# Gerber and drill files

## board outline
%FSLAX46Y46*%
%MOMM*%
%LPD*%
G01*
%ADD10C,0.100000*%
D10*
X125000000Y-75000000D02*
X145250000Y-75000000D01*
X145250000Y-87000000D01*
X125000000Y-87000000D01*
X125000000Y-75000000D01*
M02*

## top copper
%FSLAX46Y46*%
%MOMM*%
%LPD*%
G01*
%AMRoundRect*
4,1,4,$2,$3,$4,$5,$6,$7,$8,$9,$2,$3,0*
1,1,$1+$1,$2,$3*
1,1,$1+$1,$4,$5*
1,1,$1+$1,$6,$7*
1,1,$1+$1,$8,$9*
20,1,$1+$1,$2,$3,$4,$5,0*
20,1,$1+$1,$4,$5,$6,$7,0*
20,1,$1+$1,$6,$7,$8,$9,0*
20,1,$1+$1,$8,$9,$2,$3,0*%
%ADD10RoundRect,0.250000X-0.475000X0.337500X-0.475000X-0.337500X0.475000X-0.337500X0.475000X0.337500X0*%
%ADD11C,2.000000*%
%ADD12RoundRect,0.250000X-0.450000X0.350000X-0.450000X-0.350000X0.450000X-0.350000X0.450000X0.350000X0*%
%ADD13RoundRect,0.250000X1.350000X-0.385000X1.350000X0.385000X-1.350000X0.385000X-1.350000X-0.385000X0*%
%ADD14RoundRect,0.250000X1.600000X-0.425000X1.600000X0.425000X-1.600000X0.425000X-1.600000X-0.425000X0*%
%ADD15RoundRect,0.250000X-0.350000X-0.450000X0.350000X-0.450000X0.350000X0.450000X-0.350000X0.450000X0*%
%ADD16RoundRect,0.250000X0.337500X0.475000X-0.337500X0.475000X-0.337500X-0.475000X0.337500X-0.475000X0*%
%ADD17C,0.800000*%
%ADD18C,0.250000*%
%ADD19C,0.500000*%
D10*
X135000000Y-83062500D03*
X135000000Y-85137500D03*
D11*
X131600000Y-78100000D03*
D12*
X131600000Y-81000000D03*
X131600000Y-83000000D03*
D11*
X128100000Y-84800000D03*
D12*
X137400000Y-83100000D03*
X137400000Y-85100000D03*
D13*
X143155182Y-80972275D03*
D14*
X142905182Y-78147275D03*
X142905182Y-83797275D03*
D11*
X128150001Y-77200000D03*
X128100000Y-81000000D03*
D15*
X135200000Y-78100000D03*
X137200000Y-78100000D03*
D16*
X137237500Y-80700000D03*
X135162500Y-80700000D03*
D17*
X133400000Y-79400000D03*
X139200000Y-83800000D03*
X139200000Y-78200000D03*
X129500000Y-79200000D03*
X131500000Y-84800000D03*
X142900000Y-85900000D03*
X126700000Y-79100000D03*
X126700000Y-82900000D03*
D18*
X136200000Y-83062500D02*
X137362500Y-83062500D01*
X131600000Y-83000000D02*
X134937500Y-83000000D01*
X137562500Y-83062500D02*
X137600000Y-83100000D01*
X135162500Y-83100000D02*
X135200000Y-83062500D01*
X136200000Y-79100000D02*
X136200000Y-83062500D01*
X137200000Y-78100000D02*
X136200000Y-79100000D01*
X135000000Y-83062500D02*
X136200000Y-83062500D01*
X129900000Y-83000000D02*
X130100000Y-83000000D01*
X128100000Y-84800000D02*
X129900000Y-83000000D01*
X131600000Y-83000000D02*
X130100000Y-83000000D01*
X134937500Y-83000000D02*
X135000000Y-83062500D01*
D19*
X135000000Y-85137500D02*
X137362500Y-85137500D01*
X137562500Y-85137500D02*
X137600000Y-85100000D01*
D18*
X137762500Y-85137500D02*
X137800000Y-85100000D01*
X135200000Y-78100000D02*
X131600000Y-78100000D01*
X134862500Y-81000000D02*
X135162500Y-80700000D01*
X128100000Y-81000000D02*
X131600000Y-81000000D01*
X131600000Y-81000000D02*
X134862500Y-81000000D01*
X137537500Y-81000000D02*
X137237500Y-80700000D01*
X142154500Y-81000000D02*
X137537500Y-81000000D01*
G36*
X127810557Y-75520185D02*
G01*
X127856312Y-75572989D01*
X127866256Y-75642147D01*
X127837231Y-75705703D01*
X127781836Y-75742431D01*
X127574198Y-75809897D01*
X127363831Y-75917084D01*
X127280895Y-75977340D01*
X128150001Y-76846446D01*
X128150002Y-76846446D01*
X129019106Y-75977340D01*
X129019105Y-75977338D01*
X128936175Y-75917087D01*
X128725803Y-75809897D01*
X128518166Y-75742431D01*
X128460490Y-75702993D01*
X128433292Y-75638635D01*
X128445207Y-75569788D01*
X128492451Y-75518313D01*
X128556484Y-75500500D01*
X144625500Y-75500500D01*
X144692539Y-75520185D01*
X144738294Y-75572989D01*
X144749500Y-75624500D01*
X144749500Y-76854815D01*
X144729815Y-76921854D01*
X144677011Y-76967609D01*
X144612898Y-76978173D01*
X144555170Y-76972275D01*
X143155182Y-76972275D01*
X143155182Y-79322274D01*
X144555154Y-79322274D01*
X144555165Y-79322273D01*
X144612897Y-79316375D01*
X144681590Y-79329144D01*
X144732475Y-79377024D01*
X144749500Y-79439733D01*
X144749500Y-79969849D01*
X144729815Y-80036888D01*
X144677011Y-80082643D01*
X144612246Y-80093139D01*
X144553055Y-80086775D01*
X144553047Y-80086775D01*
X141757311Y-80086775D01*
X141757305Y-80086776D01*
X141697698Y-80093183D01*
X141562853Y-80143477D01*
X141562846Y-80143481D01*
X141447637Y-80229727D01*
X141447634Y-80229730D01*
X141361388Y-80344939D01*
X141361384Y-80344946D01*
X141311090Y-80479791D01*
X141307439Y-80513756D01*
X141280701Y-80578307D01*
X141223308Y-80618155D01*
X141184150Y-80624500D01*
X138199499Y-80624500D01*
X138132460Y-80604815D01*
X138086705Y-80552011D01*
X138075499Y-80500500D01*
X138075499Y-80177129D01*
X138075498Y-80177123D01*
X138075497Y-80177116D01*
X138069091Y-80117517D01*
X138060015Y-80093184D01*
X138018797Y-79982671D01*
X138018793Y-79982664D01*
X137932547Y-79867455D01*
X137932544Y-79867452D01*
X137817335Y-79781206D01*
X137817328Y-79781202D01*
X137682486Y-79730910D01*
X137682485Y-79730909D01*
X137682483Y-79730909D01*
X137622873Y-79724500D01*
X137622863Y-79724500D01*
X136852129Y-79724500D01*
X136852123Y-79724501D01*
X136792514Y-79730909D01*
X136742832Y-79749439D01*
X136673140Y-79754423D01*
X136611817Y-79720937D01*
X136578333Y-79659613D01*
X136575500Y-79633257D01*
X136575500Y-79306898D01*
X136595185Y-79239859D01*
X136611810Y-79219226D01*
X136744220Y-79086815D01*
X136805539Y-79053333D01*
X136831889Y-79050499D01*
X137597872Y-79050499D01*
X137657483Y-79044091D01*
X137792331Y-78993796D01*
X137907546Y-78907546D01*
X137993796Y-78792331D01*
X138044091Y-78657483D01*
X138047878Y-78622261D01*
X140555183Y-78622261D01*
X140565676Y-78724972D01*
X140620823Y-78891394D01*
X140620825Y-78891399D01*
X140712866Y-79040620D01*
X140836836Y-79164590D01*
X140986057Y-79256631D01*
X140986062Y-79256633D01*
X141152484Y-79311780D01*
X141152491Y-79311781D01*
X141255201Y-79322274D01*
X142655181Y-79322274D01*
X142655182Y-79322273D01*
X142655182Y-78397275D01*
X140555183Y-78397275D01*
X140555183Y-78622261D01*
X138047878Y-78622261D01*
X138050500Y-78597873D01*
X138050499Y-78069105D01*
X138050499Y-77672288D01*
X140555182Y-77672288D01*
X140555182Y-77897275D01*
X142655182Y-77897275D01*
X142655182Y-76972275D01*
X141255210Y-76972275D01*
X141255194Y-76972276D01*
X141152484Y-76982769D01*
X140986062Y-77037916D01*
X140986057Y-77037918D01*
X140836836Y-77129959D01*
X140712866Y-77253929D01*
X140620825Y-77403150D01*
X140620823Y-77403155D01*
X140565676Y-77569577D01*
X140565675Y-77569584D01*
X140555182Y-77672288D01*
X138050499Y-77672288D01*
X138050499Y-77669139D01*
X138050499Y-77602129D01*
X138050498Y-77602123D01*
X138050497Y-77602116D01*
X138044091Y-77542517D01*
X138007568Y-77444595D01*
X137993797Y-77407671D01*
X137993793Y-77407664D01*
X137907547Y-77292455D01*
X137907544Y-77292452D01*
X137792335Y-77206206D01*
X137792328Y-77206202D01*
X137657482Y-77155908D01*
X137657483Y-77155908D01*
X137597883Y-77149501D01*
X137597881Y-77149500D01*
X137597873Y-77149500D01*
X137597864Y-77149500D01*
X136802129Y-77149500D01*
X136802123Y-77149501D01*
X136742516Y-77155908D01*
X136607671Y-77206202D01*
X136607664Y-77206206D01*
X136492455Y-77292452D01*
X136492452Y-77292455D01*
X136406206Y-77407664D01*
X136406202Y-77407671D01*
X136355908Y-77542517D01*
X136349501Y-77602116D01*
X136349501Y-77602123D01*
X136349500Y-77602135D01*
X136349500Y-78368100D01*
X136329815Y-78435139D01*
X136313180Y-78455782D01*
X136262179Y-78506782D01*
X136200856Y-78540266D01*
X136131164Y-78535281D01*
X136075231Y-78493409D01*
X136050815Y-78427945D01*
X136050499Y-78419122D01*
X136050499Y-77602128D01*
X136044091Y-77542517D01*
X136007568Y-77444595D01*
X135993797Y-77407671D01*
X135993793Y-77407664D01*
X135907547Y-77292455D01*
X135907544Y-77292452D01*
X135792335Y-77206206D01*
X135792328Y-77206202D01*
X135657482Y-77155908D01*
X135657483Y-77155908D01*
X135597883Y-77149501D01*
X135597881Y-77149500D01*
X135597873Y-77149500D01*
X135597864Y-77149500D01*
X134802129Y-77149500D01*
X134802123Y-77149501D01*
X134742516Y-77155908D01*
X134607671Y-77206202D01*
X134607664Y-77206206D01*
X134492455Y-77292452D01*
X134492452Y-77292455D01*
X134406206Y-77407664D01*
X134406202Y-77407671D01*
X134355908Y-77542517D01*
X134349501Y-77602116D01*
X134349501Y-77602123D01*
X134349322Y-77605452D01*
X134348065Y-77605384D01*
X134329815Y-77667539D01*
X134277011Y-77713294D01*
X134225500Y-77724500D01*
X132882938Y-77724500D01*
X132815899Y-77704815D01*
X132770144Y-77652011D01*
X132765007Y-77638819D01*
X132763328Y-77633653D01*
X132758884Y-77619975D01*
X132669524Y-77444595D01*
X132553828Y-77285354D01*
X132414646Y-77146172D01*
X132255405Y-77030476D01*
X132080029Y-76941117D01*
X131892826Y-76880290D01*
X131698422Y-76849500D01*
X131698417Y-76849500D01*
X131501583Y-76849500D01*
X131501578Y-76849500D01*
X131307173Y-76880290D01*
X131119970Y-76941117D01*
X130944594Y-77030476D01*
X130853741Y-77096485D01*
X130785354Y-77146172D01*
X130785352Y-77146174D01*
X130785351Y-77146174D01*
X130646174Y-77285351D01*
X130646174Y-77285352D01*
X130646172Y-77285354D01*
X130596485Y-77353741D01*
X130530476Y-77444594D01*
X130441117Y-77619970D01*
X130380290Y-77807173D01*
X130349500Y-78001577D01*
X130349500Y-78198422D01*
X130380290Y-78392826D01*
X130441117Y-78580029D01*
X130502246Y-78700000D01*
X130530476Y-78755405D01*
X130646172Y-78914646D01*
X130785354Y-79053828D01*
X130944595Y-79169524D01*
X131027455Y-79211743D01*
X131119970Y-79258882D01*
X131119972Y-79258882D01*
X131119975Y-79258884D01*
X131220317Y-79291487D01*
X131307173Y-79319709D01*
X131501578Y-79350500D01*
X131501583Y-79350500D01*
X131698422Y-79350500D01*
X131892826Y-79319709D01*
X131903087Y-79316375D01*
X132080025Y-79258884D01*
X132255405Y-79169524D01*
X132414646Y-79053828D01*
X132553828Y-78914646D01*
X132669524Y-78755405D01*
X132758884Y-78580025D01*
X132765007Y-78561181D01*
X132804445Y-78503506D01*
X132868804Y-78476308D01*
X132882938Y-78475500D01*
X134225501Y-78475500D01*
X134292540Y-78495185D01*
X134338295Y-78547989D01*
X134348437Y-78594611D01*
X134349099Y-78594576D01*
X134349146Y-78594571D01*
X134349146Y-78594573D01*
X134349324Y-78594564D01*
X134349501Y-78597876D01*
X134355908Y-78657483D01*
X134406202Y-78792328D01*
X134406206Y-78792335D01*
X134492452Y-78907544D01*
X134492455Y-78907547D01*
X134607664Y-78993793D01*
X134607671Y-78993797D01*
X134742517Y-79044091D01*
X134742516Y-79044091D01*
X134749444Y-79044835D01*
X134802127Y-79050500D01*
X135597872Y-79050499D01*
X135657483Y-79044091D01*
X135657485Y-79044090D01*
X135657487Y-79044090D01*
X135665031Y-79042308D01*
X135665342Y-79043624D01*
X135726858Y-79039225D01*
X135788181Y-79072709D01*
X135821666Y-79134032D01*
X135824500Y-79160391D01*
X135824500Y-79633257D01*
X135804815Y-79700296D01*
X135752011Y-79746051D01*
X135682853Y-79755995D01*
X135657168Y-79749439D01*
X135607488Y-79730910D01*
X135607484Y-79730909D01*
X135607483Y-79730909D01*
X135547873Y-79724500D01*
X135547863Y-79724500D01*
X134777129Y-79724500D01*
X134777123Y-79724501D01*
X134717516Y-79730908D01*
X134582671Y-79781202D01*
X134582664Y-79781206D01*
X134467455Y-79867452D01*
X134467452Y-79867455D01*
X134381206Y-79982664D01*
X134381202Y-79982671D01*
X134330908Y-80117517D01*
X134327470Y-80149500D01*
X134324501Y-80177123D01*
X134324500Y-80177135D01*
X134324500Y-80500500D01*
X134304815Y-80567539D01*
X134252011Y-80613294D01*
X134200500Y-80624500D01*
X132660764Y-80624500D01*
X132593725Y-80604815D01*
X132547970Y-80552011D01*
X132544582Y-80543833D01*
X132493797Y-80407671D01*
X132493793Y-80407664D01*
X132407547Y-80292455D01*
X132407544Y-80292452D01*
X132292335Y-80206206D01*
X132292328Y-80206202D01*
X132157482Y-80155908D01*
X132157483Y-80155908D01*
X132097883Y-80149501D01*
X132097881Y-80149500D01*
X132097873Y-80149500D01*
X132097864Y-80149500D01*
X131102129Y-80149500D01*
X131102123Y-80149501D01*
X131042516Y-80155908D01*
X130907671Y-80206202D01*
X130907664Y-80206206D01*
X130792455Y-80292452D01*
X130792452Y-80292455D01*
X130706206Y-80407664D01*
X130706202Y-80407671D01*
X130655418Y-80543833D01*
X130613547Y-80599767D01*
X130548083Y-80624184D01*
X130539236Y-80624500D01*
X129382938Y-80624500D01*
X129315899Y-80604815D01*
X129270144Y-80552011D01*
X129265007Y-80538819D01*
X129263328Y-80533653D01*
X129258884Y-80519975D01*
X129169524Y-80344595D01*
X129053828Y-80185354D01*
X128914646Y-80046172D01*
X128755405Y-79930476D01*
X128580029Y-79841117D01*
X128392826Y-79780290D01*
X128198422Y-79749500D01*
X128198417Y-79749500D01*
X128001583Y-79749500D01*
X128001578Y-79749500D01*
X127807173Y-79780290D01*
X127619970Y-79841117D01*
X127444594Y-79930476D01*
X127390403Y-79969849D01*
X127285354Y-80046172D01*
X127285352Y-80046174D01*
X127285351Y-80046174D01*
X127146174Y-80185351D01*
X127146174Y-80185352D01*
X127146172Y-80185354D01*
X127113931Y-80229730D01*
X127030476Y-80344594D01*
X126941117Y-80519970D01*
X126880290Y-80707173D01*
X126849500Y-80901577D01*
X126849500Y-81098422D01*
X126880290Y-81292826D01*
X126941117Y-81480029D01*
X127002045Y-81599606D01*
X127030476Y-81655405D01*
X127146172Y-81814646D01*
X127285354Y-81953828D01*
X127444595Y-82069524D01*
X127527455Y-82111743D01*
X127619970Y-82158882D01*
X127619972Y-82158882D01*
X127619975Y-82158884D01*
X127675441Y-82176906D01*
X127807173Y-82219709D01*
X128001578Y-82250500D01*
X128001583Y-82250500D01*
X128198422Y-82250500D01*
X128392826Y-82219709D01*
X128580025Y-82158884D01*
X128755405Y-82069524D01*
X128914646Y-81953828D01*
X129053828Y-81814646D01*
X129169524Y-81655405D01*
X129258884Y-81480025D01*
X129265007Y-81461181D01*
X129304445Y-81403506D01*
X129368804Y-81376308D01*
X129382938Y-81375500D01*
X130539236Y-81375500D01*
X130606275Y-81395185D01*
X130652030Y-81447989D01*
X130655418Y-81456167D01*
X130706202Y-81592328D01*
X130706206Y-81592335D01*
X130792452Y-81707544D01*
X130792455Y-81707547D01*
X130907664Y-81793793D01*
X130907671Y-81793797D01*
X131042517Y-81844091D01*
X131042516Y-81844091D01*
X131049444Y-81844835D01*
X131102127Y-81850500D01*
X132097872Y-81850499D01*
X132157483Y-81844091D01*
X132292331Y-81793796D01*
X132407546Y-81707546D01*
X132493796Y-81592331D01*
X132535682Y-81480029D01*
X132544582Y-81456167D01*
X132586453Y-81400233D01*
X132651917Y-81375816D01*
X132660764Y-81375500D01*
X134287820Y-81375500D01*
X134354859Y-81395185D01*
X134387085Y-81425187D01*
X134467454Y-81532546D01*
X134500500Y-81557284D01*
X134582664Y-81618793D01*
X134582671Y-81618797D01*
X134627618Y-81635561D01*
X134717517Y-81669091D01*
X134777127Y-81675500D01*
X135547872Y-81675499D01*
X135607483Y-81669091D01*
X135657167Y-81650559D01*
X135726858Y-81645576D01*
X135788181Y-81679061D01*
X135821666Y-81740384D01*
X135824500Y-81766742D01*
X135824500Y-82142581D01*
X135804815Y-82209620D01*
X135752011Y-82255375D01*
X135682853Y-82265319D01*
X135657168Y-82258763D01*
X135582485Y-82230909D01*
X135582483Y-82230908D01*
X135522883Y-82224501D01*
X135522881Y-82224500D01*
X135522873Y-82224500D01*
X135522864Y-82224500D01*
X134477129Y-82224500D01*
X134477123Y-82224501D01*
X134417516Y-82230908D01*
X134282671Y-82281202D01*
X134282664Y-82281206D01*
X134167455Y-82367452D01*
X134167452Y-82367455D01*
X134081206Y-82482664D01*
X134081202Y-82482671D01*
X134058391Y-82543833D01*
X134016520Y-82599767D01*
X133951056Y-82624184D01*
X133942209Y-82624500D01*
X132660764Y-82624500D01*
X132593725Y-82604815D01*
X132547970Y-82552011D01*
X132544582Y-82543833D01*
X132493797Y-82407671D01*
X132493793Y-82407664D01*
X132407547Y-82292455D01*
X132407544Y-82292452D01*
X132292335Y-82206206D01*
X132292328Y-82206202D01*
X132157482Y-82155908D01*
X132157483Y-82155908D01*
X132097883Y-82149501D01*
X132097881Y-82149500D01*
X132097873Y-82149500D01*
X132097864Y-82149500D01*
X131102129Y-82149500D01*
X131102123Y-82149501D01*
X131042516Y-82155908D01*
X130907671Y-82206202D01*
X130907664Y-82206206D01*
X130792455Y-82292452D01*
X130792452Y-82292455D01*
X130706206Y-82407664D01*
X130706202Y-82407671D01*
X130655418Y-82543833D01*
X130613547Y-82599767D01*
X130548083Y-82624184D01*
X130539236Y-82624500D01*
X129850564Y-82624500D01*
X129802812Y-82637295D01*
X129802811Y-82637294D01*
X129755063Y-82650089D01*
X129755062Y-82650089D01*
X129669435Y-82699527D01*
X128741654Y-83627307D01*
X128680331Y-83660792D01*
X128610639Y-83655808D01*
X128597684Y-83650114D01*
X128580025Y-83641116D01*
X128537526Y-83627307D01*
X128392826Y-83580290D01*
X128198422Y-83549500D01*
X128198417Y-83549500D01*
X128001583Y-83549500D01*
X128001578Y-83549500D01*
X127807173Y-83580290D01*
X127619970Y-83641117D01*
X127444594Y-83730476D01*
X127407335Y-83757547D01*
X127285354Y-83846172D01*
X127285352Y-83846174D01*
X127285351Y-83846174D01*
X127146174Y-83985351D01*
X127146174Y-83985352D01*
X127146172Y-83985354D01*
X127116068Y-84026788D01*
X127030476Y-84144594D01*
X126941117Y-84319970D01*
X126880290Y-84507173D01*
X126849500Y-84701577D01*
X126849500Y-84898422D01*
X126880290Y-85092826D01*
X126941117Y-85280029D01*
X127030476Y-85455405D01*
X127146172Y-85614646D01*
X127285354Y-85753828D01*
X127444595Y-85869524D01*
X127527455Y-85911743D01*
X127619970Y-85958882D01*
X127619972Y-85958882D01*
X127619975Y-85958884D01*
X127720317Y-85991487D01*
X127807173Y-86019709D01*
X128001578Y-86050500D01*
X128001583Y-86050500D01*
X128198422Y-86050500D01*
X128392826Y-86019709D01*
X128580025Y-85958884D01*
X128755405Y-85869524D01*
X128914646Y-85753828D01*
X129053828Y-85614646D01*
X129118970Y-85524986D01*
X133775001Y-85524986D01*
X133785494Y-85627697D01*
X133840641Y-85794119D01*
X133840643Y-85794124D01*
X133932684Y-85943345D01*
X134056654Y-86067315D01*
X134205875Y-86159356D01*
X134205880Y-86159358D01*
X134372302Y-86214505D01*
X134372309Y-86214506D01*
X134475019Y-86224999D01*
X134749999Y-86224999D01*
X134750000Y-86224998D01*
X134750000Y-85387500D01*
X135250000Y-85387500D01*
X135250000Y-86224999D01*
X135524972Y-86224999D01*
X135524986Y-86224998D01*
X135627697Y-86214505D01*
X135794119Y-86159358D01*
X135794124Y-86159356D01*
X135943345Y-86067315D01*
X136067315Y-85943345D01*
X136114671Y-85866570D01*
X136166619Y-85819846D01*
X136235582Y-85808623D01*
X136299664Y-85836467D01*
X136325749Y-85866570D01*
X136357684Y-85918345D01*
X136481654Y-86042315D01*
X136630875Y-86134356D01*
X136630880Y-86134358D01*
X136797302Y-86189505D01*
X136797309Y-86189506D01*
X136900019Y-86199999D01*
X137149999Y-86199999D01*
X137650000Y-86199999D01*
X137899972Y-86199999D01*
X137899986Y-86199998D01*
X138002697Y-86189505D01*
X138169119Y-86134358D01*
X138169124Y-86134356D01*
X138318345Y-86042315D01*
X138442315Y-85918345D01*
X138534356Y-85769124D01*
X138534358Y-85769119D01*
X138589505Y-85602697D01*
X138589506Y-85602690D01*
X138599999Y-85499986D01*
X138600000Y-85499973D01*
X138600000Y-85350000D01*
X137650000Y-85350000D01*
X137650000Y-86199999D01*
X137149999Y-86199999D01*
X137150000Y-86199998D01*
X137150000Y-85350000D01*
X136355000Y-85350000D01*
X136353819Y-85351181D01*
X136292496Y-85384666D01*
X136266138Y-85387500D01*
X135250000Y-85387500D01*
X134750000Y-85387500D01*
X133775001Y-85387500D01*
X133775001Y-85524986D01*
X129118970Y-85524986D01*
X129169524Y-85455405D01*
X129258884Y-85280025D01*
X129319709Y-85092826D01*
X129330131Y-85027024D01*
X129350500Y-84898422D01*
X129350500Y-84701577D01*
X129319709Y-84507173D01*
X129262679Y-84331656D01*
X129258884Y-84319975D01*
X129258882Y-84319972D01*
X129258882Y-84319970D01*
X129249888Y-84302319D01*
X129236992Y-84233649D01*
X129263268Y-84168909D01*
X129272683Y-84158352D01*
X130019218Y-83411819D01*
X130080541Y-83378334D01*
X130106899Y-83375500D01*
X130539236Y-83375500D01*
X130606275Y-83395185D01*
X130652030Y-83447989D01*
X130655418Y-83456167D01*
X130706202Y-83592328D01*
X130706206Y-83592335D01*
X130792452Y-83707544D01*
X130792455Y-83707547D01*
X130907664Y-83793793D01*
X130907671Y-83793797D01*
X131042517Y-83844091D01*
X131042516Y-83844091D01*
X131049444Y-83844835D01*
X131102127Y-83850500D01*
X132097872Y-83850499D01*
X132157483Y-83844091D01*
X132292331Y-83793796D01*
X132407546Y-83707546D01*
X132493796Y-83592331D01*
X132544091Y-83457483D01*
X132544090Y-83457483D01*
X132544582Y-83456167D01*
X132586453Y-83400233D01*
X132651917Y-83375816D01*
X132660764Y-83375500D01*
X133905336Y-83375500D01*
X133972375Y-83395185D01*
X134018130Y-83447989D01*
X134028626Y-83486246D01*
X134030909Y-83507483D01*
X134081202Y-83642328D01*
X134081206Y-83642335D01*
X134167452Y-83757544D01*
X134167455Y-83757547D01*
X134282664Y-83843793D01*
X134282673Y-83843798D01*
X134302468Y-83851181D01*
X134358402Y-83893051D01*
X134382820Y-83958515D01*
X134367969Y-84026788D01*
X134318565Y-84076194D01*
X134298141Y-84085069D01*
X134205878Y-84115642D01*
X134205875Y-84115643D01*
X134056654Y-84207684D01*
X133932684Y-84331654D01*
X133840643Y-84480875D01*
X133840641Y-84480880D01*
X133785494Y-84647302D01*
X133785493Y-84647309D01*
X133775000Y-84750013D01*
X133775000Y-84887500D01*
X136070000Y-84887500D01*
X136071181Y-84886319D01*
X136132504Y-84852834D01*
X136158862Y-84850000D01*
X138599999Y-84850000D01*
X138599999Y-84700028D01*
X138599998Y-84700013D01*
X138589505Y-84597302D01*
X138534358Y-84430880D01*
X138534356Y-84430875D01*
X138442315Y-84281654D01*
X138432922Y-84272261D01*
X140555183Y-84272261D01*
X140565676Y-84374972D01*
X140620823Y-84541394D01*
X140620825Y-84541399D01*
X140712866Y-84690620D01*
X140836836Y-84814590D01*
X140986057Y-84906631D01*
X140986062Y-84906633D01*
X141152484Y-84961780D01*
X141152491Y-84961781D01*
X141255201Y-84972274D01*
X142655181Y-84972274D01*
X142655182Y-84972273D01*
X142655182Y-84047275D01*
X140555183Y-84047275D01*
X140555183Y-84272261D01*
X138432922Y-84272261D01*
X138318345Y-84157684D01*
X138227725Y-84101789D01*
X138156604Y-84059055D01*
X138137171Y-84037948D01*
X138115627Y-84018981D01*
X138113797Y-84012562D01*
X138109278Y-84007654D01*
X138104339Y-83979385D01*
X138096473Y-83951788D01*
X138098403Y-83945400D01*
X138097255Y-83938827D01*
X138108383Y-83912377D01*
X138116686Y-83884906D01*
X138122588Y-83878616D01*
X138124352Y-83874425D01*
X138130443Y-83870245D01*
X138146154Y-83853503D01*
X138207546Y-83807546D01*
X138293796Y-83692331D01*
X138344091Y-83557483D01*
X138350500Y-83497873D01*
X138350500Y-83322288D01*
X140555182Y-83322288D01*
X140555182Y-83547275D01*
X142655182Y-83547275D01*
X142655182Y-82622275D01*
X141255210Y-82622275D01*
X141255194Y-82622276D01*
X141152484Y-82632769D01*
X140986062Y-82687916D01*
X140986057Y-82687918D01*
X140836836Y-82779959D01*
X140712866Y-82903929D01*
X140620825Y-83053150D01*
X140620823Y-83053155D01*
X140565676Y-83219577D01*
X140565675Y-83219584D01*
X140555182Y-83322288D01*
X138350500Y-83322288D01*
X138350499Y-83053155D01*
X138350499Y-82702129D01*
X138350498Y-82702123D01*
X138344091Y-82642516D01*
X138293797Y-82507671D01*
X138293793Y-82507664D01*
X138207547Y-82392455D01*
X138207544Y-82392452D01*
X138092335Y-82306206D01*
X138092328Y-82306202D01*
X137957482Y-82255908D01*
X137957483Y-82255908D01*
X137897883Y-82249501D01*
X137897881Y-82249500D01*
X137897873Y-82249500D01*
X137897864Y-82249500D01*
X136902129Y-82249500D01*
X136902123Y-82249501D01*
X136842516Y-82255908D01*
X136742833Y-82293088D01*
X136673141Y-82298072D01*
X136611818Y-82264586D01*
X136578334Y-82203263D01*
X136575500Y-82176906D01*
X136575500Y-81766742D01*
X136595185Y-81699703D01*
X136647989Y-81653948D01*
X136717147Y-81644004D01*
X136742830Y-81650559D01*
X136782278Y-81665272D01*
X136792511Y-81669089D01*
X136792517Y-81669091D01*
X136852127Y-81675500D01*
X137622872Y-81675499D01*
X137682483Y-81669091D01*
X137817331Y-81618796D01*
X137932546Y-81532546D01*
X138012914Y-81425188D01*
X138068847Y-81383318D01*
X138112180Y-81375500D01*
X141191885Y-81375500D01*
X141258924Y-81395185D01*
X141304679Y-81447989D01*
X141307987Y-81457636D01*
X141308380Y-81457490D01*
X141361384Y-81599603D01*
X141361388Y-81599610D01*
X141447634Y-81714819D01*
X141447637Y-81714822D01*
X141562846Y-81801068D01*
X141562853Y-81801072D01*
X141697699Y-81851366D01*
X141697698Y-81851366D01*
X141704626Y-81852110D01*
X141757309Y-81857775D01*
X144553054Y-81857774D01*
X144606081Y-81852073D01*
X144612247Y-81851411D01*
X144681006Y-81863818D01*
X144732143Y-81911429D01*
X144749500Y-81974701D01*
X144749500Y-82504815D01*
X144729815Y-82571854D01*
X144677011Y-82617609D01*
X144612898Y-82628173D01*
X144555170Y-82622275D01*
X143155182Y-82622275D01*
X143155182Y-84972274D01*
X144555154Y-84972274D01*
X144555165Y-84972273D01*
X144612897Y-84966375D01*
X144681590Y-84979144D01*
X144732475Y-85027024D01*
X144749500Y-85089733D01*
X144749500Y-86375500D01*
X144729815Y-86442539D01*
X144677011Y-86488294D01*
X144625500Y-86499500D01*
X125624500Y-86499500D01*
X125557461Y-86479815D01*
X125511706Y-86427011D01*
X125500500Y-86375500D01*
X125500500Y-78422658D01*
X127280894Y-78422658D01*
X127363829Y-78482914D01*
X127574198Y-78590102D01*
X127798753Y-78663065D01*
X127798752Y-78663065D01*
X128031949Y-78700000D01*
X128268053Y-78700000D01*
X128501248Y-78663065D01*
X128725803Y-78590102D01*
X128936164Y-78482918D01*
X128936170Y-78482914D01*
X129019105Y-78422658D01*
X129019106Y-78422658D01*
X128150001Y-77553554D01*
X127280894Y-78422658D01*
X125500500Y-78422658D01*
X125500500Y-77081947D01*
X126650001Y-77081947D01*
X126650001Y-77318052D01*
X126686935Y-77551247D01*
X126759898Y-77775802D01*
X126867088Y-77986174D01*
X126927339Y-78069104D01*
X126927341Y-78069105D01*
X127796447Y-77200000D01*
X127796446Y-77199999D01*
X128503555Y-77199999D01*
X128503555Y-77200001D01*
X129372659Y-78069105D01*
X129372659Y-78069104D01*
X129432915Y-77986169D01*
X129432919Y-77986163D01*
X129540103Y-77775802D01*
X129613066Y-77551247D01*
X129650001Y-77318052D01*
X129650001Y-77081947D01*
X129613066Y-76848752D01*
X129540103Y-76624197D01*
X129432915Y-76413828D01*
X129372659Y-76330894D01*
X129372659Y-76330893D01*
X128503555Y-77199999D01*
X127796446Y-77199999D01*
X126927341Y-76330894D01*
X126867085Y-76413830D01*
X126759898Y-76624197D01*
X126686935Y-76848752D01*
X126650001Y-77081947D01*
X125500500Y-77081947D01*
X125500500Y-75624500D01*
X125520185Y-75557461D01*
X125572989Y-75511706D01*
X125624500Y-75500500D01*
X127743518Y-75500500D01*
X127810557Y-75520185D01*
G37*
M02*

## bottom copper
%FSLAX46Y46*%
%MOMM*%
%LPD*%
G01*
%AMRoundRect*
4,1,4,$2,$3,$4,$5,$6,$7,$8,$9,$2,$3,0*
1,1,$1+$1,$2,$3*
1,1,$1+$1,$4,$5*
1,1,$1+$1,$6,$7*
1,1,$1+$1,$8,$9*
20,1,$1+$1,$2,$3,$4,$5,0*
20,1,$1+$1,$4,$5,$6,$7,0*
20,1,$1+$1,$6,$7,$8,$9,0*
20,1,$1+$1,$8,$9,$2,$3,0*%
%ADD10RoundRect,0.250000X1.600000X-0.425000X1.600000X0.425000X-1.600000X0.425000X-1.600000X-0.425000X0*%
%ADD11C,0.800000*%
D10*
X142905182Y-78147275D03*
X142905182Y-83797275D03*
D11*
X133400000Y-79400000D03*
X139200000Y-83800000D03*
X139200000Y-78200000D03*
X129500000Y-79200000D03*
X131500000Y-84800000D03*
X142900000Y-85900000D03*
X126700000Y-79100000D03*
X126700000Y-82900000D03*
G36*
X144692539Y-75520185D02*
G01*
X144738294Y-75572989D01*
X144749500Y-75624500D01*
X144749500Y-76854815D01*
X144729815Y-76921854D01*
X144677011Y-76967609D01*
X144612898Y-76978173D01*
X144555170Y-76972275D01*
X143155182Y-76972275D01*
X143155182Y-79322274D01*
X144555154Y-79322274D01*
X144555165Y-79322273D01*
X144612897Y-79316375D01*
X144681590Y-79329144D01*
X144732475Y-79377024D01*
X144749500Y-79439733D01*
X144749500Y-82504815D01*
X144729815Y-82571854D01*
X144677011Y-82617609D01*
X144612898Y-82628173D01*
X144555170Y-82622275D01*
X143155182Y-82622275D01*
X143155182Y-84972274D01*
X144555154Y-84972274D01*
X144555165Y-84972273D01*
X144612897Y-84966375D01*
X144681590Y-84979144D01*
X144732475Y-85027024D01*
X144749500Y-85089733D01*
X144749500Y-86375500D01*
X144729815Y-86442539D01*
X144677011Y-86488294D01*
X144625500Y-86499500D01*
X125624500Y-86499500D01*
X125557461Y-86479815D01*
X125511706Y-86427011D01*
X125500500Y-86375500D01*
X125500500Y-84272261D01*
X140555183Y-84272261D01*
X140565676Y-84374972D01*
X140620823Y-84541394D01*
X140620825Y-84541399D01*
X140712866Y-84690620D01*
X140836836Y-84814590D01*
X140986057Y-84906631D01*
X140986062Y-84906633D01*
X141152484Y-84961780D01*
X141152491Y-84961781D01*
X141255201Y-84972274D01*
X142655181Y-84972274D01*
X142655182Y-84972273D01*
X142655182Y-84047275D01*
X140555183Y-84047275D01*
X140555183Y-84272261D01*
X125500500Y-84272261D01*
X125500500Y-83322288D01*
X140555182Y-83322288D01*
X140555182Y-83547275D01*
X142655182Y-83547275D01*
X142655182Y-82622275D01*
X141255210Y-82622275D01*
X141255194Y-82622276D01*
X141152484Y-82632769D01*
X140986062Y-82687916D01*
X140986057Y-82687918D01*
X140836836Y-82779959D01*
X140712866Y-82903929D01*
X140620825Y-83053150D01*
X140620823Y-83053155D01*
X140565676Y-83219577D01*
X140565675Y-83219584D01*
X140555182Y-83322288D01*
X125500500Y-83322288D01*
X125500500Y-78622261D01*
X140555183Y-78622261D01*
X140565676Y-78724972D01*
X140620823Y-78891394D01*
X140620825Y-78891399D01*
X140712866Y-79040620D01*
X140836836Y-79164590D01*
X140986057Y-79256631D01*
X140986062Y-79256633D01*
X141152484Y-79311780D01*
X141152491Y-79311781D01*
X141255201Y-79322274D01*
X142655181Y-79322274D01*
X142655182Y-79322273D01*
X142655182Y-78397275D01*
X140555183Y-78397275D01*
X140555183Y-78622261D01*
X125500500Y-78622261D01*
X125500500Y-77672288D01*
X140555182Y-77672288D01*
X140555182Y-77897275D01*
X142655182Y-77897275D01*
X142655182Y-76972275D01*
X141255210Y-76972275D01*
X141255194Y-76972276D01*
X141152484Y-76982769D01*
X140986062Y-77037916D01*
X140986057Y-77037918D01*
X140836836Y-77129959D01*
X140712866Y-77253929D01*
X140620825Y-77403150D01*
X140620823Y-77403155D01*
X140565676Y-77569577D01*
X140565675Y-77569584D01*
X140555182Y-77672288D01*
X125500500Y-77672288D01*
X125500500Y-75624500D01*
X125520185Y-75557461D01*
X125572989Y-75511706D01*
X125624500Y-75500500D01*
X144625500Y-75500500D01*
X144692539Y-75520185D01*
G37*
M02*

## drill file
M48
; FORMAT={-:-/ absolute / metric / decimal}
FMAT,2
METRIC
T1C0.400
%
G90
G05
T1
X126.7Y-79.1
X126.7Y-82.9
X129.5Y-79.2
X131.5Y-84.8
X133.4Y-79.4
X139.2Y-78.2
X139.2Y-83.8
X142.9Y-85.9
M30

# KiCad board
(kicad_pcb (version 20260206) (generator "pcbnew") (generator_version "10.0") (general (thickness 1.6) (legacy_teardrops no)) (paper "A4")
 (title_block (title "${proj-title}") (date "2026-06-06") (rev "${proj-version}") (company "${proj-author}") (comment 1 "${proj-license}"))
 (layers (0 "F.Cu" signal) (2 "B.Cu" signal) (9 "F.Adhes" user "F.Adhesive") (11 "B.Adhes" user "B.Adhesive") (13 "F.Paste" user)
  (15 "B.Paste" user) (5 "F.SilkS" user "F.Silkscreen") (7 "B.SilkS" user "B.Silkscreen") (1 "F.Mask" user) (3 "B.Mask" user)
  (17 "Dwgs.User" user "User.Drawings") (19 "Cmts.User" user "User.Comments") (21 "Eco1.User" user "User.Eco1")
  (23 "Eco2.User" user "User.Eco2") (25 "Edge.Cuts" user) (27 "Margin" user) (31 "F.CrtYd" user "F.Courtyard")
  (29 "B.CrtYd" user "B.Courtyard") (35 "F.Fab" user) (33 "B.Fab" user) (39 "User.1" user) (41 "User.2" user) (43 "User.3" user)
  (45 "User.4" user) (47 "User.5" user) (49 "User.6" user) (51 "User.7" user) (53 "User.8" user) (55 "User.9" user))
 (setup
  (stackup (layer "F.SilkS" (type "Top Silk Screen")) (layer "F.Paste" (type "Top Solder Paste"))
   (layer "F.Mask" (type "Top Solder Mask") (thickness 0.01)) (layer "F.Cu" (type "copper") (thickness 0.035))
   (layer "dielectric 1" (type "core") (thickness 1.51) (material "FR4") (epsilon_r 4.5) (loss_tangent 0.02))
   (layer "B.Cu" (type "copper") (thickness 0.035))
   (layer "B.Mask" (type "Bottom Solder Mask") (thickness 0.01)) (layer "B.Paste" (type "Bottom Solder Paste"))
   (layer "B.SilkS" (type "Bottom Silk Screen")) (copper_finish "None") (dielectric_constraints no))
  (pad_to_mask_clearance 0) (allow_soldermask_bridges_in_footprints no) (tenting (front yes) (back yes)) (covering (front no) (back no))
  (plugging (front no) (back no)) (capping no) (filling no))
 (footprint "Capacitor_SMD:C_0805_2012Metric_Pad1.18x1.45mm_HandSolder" (layer "F.Cu") (at 135 84.1 -90)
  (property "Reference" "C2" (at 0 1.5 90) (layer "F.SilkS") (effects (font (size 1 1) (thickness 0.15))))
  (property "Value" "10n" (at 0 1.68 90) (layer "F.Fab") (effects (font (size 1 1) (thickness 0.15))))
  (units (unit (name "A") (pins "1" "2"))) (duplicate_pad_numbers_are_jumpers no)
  (pad "1" smd roundrect (at -1.0375 0 270) (size 1.175 1.45) (layers "F.Cu" "F.Mask" "F.Paste") (roundrect_rratio 0.2127659574)
   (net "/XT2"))
  (pad "2" smd roundrect (at 1.0375 0 270) (size 1.175 1.45) (layers "F.Cu" "F.Mask" "F.Paste") (roundrect_rratio 0.2127659574) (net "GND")))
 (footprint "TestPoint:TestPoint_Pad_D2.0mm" (layer "F.Cu") (at 131.6 78.1)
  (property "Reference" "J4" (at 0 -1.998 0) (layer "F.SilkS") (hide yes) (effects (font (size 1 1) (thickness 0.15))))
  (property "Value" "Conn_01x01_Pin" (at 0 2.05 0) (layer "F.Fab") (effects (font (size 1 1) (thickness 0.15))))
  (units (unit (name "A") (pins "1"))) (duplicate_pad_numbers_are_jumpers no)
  (pad "1" smd circle (at 0 0) (size 2 2) (layers "F.Cu" "F.Mask") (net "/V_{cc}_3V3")))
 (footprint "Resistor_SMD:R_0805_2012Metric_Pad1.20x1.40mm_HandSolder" (layer "F.Cu") (at 131.6 82 -90)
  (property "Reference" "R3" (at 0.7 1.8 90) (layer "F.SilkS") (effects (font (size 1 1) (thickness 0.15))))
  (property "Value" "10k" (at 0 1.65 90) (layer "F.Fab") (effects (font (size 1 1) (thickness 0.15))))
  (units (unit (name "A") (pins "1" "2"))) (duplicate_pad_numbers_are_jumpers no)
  (pad "1" smd roundrect (at -1 0 270) (size 1.2 1.4) (layers "F.Cu" "F.Mask" "F.Paste") (roundrect_rratio 0.2083333333) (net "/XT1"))
  (pad "2" smd roundrect (at 1 0 270) (size 1.2 1.4) (layers "F.Cu" "F.Mask" "F.Paste") (roundrect_rratio 0.2083333333) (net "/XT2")))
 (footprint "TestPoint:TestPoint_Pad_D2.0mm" (layer "F.Cu") (at 128.1 84.8)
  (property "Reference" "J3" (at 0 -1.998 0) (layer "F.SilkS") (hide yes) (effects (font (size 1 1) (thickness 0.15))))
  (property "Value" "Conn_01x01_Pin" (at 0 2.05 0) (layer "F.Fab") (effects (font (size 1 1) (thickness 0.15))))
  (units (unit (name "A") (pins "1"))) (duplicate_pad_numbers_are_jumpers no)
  (pad "1" smd circle (at 0 0) (size 2 2) (layers "F.Cu" "F.Mask") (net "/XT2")))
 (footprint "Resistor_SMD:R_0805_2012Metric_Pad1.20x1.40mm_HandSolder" (layer "F.Cu") (at 137.4 84.1 -90)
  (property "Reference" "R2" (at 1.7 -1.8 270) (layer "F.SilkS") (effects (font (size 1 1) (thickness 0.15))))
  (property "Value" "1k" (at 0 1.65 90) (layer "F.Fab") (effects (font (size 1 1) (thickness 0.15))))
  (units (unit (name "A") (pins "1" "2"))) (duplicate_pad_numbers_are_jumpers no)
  (pad "1" smd roundrect (at -1 0 270) (size 1.2 1.4) (layers "F.Cu" "F.Mask" "F.Paste") (roundrect_rratio 0.2083333333) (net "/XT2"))
  (pad "2" smd roundrect (at 1 0 270) (size 1.2 1.4) (layers "F.Cu" "F.Mask" "F.Paste") (roundrect_rratio 0.2083333333) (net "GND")))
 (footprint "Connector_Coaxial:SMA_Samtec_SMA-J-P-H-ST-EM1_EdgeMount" (layer "F.Cu") (at 143.155182 80.972275)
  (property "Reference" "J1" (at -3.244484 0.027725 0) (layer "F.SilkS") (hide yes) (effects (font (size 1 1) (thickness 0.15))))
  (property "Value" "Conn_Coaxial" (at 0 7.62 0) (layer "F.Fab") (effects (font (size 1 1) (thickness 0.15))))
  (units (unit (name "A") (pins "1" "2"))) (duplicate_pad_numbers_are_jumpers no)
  (pad "1" smd roundrect (at 0 0 90) (size 1.27 3.2) (layers "F.Cu" "F.Mask") (roundrect_rratio 0.1968503937) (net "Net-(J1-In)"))
  (pad "2" smd roundrect (at -0.25 -2.825 90) (size 1.35 3.7) (layers "F.Cu" "F.Mask") (roundrect_rratio 0.1851851852) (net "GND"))
  (pad "2" smd roundrect (at -0.25 -2.825 90) (size 1.35 3.7) (layers "B.Cu" "B.Mask") (roundrect_rratio 0.1851851852) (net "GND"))
  (pad "2" smd roundrect (at -0.25 2.825 90) (size 1.35 3.7) (layers "F.Cu" "F.Mask") (roundrect_rratio 0.1851851852) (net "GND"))
  (pad "2" smd roundrect (at -0.25 2.825 90) (size 1.35 3.7) (layers "B.Cu" "B.Mask") (roundrect_rratio 0.1851851852) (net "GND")))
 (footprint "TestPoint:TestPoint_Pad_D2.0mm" (layer "F.Cu") (at 128.150001 77.2)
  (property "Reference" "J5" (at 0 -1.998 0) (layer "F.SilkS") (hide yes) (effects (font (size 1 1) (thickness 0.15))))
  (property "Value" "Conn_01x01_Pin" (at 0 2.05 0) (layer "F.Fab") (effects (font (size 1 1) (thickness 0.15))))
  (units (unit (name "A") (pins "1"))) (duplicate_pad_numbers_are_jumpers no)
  (pad "1" smd circle (at 0 0) (size 2 2) (layers "F.Cu" "F.Mask") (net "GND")))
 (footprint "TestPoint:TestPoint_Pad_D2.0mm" (layer "F.Cu") (at 128.1 81)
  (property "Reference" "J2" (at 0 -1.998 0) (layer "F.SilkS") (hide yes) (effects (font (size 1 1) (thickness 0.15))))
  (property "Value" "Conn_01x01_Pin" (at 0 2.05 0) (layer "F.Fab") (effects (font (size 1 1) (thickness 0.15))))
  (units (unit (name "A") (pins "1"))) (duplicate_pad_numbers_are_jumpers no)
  (pad "1" smd circle (at 0 0) (size 2 2) (layers "F.Cu" "F.Mask") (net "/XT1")))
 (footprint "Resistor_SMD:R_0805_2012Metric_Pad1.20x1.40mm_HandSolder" (layer "F.Cu") (at 136.2 78.1)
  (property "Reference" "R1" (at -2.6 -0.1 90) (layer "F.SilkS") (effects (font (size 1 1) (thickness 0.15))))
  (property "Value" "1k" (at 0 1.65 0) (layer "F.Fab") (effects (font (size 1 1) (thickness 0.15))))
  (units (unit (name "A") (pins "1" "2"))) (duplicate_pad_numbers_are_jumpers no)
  (pad "1" smd roundrect (at -1 0) (size 1.2 1.4) (layers "F.Cu" "F.Mask" "F.Paste") (roundrect_rratio 0.2083333333) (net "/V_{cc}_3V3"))
  (pad "2" smd roundrect (at 1 0) (size 1.2 1.4) (layers "F.Cu" "F.Mask" "F.Paste") (roundrect_rratio 0.2083333333) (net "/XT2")))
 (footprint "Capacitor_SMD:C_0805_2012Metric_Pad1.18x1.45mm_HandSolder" (layer "F.Cu") (at 136.2 80.7 180)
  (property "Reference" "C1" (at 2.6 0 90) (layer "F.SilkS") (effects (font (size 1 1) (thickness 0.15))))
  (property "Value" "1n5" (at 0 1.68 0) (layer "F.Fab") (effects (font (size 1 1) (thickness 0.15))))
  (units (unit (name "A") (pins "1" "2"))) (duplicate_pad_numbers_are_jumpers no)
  (pad "1" smd roundrect (at -1.0375 0 180) (size 1.175 1.45) (layers "F.Cu" "F.Mask" "F.Paste") (roundrect_rratio 0.2127659574)
   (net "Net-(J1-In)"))
  (pad "2" smd roundrect (at 1.0375 0 180) (size 1.175 1.45) (layers "F.Cu" "F.Mask" "F.Paste") (roundrect_rratio 0.2127659574) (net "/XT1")))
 (gr_rect (start 125 75) (end 145.25 87) (stroke (width 0.1) (type default)) (fill no) (layer "Edge.Cuts"))
 (segment (start 136.2 83.0625) (end 137.3625 83.0625) (width 0.25) (layer "F.Cu") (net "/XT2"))
 (segment (start 131.6 83) (end 134.9375 83) (width 0.25) (layer "F.Cu") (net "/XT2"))
 (segment (start 137.5625 83.0625) (end 137.6 83.1) (width 0.25) (layer "F.Cu") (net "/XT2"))
 (segment (start 135.1625 83.1) (end 135.2 83.0625) (width 0.25) (layer "F.Cu") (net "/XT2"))
 (segment (start 136.2 79.1) (end 136.2 83.0625) (width 0.25) (layer "F.Cu") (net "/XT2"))
 (segment (start 137.2 78.1) (end 136.2 79.1) (width 0.25) (layer "F.Cu") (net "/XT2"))
 (segment (start 135 83.0625) (end 136.2 83.0625) (width 0.25) (layer "F.Cu") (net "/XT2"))
 (segment (start 129.9 83) (end 130.1 83) (width 0.25) (layer "F.Cu") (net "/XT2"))
 (segment (start 128.1 84.8) (end 129.9 83) (width 0.25) (layer "F.Cu") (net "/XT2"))
 (segment (start 131.6 83) (end 130.1 83) (width 0.25) (layer "F.Cu") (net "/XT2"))
 (segment (start 134.9375 83) (end 135 83.0625) (width 0.25) (layer "F.Cu") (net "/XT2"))
 (segment (start 135 85.1375) (end 137.3625 85.1375) (width 0.5) (layer "F.Cu") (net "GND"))
 (segment (start 137.5625 85.1375) (end 137.6 85.1) (width 0.5) (layer "F.Cu") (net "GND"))
 (segment (start 137.7625 85.1375) (end 137.8 85.1) (width 0.25) (layer "F.Cu") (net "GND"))
 (via (at 133.4 79.4) (size 0.8) (drill 0.4) (layers "F.Cu" "B.Cu") (free yes) (capping no) (covering (front no) (back no))
  (plugging (front no) (back no)) (filling no) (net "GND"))
 (via (at 139.2 83.8) (size 0.8) (drill 0.4) (layers "F.Cu" "B.Cu") (free yes) (capping no) (covering (front no) (back no))
  (plugging (front no) (back no)) (filling no) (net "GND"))
 (via (at 139.2 78.2) (size 0.8) (drill 0.4) (layers "F.Cu" "B.Cu") (free yes) (capping no) (covering (front no) (back no))
  (plugging (front no) (back no)) (filling no) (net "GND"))
 (via (at 129.5 79.2) (size 0.8) (drill 0.4) (layers "F.Cu" "B.Cu") (free yes) (capping no) (covering (front no) (back no))
  (plugging (front no) (back no)) (filling no) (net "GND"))
 (via (at 131.5 84.8) (size 0.8) (drill 0.4) (layers "F.Cu" "B.Cu") (free yes) (capping no) (covering (front no) (back no))
  (plugging (front no) (back no)) (filling no) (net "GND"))
 (via (at 142.9 85.9) (size 0.8) (drill 0.4) (layers "F.Cu" "B.Cu") (free yes) (capping no) (covering (front no) (back no))
  (plugging (front no) (back no)) (filling no) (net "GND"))
 (via (at 126.7 79.1) (size 0.8) (drill 0.4) (layers "F.Cu" "B.Cu") (free yes) (capping no) (covering (front no) (back no))
  (plugging (front no) (back no)) (filling no) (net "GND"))
 (via (at 126.7 82.9) (size 0.8) (drill 0.4) (layers "F.Cu" "B.Cu") (free yes) (capping no) (covering (front no) (back no))
  (plugging (front no) (back no)) (filling no) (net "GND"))
 (segment (start 135.2 78.1) (end 131.6 78.1) (width 0.25) (layer "F.Cu") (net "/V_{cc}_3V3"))
 (segment (start 134.8625 81) (end 135.1625 80.7) (width 0.25) (layer "F.Cu") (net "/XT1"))
 (segment (start 128.1 81) (end 131.6 81) (width 0.25) (layer "F.Cu") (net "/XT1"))
 (segment (start 131.6 81) (end 134.8625 81) (width 0.25) (layer "F.Cu") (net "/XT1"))
 (segment (start 137.5375 81) (end 137.2375 80.7) (width 0.25) (layer "F.Cu") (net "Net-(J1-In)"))
 (segment (start 142.1545 81) (end 137.5375 81) (width 0.25) (layer "F.Cu") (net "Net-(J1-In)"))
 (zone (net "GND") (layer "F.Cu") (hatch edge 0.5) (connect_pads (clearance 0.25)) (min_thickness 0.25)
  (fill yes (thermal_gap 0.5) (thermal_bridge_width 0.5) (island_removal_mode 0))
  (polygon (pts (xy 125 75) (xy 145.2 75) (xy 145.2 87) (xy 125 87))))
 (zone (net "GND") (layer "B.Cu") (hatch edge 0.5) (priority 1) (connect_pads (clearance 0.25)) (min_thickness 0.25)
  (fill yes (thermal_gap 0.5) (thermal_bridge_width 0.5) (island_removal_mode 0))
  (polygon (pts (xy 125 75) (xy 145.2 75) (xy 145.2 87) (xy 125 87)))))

